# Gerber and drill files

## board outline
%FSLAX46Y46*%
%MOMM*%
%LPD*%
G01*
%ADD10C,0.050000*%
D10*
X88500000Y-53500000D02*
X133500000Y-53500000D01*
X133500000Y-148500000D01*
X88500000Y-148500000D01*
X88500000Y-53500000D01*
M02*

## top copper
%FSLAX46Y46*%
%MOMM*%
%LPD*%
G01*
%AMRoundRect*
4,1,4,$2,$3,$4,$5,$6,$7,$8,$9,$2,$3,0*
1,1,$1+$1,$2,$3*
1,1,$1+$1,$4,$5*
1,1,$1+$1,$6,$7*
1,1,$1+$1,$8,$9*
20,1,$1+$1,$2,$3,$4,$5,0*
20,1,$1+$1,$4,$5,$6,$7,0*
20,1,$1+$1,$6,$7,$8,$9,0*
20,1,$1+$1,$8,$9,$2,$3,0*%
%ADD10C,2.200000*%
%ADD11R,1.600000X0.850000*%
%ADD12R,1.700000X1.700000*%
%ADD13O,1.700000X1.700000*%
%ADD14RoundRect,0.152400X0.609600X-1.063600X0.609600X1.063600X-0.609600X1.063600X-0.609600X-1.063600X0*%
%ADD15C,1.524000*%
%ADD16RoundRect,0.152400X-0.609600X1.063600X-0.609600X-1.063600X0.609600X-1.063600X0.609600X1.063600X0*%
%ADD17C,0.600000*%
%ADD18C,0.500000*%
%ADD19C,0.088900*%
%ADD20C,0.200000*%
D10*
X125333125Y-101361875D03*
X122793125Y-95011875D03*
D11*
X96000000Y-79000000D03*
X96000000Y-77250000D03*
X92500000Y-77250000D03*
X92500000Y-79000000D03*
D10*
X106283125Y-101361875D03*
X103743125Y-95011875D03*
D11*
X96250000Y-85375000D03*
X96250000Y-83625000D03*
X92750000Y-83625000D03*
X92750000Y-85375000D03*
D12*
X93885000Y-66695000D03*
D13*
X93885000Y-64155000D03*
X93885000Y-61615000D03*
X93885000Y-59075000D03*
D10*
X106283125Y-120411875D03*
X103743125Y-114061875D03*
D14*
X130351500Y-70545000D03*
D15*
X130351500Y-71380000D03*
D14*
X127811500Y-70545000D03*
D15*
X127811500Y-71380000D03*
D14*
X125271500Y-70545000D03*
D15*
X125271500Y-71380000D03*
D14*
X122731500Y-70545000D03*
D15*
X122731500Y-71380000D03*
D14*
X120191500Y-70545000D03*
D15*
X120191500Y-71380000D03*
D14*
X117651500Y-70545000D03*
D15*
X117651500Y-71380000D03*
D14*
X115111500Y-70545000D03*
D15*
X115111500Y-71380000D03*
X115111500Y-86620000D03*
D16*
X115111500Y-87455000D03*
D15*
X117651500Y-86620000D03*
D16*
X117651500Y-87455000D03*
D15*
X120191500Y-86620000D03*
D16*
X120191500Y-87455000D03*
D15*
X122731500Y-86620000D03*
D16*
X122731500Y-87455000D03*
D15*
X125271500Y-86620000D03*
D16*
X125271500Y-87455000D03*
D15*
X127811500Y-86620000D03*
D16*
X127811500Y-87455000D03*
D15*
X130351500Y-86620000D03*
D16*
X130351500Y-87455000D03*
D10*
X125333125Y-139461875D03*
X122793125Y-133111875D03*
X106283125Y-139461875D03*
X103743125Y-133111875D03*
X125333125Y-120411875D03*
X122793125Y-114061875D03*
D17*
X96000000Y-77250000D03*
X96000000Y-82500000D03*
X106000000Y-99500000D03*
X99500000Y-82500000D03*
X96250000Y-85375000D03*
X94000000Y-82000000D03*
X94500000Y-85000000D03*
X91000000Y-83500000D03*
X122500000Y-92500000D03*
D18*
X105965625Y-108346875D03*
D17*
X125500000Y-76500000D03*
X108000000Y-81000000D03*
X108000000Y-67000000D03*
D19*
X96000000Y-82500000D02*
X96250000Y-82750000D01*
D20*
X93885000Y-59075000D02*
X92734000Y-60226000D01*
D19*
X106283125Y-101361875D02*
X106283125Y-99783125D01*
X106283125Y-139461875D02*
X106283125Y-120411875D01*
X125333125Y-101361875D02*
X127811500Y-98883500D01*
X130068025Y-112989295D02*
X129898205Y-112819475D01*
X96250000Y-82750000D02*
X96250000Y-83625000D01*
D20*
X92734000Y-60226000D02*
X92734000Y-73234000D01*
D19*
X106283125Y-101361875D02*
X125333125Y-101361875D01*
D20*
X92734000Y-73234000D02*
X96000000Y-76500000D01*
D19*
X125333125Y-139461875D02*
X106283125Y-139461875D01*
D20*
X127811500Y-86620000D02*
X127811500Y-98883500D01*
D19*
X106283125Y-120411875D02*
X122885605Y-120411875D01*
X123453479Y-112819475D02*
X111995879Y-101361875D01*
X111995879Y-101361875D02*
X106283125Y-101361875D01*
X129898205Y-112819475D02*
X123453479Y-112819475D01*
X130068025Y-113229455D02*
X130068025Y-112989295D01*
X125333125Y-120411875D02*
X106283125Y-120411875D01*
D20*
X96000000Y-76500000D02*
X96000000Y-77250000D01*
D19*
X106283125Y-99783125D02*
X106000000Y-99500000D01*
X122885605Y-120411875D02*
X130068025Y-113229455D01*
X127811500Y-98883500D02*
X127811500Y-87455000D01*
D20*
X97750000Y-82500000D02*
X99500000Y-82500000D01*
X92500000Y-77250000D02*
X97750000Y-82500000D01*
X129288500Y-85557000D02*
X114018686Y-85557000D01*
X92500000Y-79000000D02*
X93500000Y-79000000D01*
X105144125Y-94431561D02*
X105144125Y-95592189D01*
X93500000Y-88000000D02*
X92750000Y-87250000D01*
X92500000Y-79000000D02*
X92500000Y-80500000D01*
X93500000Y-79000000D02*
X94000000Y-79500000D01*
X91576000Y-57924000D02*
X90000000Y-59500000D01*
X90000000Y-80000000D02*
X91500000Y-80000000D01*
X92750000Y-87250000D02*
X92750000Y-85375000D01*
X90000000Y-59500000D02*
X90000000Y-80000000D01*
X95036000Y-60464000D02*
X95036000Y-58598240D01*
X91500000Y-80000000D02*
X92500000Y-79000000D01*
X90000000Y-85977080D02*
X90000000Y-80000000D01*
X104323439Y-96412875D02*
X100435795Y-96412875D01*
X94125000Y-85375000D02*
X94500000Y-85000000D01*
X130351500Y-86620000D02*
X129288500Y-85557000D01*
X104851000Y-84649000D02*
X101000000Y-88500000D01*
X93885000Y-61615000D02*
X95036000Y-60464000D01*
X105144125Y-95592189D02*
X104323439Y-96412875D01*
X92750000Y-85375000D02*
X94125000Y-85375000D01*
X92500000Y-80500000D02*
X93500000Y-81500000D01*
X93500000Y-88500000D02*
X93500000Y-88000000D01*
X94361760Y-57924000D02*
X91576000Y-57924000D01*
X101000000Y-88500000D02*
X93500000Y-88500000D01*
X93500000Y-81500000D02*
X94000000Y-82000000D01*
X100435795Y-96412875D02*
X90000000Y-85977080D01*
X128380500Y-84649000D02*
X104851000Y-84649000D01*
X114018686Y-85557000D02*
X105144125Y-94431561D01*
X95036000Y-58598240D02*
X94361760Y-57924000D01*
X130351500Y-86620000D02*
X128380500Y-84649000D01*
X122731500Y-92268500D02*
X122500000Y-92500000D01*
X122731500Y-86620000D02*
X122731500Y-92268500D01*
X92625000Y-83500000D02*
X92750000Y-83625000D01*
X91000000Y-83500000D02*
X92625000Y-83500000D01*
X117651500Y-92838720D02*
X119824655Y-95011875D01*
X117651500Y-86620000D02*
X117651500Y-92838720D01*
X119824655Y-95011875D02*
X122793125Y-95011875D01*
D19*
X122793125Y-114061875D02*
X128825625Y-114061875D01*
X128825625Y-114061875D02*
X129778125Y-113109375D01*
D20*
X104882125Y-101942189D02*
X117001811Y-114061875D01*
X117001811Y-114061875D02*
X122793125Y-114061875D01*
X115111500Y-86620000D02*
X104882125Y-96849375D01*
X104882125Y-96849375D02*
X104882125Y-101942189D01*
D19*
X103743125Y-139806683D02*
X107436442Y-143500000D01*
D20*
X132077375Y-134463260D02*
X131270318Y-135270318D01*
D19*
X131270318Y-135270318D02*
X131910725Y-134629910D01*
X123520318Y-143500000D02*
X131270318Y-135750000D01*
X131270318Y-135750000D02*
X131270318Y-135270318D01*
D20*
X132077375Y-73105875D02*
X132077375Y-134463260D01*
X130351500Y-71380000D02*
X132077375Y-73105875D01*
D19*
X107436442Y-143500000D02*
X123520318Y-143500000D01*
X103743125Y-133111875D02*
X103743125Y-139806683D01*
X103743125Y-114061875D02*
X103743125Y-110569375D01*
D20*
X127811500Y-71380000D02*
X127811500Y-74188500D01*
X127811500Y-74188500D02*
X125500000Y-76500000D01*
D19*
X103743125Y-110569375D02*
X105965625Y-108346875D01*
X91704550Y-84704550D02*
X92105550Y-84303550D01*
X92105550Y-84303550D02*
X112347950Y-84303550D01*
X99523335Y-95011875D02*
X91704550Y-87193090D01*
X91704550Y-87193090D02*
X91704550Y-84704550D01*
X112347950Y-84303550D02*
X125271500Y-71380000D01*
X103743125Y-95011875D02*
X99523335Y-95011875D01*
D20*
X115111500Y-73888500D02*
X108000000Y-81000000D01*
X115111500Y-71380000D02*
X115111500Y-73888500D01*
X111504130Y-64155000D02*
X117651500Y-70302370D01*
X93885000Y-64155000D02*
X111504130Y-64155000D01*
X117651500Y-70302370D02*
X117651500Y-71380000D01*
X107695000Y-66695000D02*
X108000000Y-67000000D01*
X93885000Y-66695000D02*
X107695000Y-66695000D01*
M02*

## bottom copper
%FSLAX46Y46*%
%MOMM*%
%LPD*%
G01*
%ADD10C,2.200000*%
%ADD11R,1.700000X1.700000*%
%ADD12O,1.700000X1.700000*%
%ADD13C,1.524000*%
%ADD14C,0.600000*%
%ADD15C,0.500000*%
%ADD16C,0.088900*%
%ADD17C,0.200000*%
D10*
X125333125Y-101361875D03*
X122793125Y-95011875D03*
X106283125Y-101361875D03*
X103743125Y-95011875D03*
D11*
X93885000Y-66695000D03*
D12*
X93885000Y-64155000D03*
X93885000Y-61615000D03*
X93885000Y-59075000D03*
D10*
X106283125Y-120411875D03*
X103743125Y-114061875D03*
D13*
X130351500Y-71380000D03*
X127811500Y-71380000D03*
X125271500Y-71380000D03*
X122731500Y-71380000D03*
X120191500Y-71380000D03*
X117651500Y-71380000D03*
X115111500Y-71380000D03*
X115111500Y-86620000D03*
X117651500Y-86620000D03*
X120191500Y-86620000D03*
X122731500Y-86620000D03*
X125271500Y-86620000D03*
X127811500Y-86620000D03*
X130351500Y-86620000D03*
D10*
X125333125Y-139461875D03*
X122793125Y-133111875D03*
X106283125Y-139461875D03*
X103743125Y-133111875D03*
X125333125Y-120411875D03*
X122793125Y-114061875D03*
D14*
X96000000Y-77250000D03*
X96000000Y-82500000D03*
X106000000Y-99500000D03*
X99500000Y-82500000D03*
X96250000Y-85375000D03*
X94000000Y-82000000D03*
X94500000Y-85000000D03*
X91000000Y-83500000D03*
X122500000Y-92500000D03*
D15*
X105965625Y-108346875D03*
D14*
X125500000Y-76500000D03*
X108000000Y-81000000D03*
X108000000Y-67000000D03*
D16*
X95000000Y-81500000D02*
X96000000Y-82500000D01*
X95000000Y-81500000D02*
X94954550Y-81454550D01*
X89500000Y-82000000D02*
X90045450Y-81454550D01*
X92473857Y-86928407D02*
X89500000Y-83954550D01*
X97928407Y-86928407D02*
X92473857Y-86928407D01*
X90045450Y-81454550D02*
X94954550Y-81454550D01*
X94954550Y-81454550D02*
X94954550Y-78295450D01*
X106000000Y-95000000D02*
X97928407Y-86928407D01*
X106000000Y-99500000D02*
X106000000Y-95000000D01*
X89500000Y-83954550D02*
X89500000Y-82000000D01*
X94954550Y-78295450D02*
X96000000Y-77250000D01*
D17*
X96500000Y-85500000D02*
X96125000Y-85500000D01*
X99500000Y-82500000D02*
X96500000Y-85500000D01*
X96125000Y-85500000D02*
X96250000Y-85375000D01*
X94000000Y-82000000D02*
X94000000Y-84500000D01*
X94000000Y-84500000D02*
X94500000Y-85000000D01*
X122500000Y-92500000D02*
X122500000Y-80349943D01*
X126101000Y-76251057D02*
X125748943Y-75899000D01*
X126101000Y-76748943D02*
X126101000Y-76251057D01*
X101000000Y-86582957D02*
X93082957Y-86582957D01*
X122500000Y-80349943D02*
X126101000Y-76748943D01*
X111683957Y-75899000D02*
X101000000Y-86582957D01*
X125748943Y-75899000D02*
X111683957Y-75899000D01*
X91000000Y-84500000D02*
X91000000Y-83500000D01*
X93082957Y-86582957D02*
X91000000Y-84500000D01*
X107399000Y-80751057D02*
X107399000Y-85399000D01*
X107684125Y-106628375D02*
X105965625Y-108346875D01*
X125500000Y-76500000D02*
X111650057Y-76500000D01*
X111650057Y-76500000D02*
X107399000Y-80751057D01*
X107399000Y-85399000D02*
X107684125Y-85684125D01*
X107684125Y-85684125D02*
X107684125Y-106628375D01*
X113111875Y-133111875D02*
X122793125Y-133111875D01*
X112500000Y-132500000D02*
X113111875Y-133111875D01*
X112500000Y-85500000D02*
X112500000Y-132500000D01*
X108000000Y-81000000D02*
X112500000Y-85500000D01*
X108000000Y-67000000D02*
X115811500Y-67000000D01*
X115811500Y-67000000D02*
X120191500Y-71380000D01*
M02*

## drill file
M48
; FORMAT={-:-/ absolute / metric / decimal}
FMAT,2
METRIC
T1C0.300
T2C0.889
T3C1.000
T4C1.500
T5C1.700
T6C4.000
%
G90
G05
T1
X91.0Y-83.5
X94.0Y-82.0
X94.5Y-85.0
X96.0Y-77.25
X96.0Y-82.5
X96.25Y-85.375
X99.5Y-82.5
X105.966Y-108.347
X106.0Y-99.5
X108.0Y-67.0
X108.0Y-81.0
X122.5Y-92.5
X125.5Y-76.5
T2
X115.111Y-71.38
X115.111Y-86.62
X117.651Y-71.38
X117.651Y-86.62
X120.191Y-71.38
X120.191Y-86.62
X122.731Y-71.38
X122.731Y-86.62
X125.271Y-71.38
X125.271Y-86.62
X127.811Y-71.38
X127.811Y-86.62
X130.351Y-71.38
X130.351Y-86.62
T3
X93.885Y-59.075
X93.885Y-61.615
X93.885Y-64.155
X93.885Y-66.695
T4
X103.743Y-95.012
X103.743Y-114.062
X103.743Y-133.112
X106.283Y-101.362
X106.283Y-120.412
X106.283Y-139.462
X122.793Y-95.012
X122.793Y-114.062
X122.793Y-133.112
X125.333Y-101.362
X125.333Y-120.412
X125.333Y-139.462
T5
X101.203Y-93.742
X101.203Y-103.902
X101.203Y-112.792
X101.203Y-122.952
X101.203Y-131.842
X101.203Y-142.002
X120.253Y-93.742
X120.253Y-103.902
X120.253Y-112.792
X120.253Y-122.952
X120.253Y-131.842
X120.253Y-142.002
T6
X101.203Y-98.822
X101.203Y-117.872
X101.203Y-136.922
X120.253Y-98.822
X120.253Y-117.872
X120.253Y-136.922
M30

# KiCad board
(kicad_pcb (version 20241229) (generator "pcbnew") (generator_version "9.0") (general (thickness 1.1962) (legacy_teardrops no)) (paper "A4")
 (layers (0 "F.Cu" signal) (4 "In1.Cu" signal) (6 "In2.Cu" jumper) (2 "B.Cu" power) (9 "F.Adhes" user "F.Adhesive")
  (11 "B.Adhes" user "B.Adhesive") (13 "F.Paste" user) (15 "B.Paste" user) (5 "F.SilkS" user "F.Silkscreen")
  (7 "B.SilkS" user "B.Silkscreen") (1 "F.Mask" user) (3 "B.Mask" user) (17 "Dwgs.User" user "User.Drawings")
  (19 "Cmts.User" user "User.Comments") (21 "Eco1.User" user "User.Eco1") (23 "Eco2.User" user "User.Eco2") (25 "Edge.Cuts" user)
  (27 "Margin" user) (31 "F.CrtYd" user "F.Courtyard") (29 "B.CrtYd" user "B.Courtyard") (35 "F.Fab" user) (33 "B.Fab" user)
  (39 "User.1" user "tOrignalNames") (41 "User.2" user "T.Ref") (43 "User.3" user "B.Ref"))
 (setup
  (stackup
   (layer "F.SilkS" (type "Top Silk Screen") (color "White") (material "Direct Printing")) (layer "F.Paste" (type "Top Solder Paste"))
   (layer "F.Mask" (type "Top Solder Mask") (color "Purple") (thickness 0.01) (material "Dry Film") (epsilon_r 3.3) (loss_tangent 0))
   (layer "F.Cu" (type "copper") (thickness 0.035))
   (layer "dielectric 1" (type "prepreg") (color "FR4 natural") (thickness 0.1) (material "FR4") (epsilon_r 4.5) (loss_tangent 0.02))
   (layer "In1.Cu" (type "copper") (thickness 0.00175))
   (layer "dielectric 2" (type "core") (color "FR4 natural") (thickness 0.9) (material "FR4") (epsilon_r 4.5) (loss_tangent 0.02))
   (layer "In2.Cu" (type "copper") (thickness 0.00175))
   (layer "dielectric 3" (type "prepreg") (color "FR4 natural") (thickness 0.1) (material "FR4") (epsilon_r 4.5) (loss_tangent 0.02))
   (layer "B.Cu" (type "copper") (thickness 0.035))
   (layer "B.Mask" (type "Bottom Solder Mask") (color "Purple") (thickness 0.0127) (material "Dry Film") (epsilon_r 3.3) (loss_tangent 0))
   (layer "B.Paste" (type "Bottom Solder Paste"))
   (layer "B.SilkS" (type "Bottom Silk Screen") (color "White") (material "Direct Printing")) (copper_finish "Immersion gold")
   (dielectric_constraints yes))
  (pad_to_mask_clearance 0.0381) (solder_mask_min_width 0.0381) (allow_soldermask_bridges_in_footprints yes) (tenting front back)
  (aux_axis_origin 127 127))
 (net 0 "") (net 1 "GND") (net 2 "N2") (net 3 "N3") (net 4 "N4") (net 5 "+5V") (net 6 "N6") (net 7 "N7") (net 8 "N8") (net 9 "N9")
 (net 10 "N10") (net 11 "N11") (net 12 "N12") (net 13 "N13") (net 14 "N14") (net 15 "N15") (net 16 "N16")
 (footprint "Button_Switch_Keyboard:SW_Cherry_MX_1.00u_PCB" (layer "F.Cu") (at 125.333125 101.361875 -90)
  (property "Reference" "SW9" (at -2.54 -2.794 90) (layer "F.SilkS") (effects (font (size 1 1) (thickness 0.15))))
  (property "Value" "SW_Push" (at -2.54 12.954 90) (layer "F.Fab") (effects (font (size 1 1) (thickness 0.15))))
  (pad "" np_thru_hole circle (at -7.62 5.08 270) (size 1.7 1.7) (drill 1.7) (layers "*.Cu" "*.Mask"))
  (pad "" np_thru_hole circle (at -2.54 5.08 270) (size 4 4) (drill 4) (layers "*.Cu" "*.Mask"))
  (pad "" np_thru_hole circle (at 2.54 5.08 270) (size 1.7 1.7) (drill 1.7) (layers "*.Cu" "*.Mask"))
  (pad "1" thru_hole circle (at 0 0 270) (size 2.2 2.2) (drill 1.5) (layers "*.Cu" "*.Mask") (remove_unused_layers no) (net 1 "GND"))
  (pad "2" thru_hole circle (at -6.35 2.54 270) (size 2.2 2.2) (drill 1.5) (layers "*.Cu" "*.Mask") (remove_unused_layers no) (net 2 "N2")))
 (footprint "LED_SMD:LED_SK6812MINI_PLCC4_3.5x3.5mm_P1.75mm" (layer "F.Cu") (at 94.25 78.125 180)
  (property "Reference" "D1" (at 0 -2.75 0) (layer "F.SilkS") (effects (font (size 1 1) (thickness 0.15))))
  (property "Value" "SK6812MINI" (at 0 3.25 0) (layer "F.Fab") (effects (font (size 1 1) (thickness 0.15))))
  (pad "1" smd rect (at -1.75 -0.875 180) (size 1.6 0.85) (layers "F.Cu" "F.Mask" "F.Paste") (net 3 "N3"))
  (pad "2" smd rect (at -1.75 0.875 180) (size 1.6 0.85) (layers "F.Cu" "F.Mask" "F.Paste") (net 1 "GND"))
  (pad "3" smd rect (at 1.75 0.875 180) (size 1.6 0.85) (layers "F.Cu" "F.Mask" "F.Paste") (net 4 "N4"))
  (pad "4" smd rect (at 1.75 -0.875 180) (size 1.6 0.85) (layers "F.Cu" "F.Mask" "F.Paste") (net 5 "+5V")))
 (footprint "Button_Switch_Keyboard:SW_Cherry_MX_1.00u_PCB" (layer "F.Cu") (at 106.283125 101.361875 -90)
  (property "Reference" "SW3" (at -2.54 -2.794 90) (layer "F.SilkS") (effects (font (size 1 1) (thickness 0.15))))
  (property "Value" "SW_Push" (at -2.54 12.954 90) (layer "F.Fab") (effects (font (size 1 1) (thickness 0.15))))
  (pad "" np_thru_hole circle (at -7.62 5.08 270) (size 1.7 1.7) (drill 1.7) (layers "*.Cu" "*.Mask"))
  (pad "" np_thru_hole circle (at -2.54 5.08 270) (size 4 4) (drill 4) (layers "*.Cu" "*.Mask"))
  (pad "" np_thru_hole circle (at 2.54 5.08 270) (size 1.7 1.7) (drill 1.7) (layers "*.Cu" "*.Mask"))
  (pad "1" thru_hole circle (at 0 0 270) (size 2.2 2.2) (drill 1.5) (layers "*.Cu" "*.Mask") (remove_unused_layers no) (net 1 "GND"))
  (pad "2" thru_hole circle (at -6.35 2.54 270) (size 2.2 2.2) (drill 1.5) (layers "*.Cu" "*.Mask") (remove_unused_layers no) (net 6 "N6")))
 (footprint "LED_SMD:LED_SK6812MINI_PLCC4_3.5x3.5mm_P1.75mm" (layer "F.Cu") (at 94.5 84.5 180)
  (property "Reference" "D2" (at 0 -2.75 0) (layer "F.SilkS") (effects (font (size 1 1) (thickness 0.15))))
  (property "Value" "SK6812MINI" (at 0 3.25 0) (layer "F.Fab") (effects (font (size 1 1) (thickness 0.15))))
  (pad "1" smd rect (at -1.75 -0.875 180) (size 1.6 0.85) (layers "F.Cu" "F.Mask" "F.Paste") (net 4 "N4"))
  (pad "2" smd rect (at -1.75 0.875 180) (size 1.6 0.85) (layers "F.Cu" "F.Mask" "F.Paste") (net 1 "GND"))
  (pad "3" smd rect (at 1.75 0.875 180) (size 1.6 0.85) (layers "F.Cu" "F.Mask" "F.Paste") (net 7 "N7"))
  (pad "4" smd rect (at 1.75 -0.875 180) (size 1.6 0.85) (layers "F.Cu" "F.Mask" "F.Paste") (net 5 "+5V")))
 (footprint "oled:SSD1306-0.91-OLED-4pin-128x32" (layer "F.Cu") (at 130.385 68.885 180)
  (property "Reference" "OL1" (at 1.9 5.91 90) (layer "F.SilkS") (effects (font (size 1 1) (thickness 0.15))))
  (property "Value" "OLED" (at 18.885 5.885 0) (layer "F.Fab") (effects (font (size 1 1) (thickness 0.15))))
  (pad "1" thru_hole rect (at 36.5 2.19 180) (size 1.7 1.7) (drill 1) (layers "*.Cu" "*.Mask") (remove_unused_layers no) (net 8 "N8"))
  (pad "2" thru_hole oval (at 36.5 4.73 180) (size 1.7 1.7) (drill 1) (layers "*.Cu" "*.Mask") (remove_unused_layers no) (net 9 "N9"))
  (pad "3" thru_hole oval (at 36.5 7.27 180) (size 1.7 1.7) (drill 1) (layers "*.Cu" "*.Mask") (remove_unused_layers no) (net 5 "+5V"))
  (pad "4" thru_hole oval (at 36.5 9.81 180) (size 1.7 1.7) (drill 1) (layers "*.Cu" "*.Mask") (remove_unused_layers no) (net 1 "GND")))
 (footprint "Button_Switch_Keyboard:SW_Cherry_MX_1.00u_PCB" (layer "F.Cu") (at 106.283125 120.411875 -90)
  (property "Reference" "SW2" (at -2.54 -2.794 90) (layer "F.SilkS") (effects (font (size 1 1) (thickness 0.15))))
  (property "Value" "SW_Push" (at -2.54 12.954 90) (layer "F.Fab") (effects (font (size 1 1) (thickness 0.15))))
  (pad "" np_thru_hole circle (at -7.62 5.08 270) (size 1.7 1.7) (drill 1.7) (layers "*.Cu" "*.Mask"))
  (pad "" np_thru_hole circle (at -2.54 5.08 270) (size 4 4) (drill 4) (layers "*.Cu" "*.Mask"))
  (pad "" np_thru_hole circle (at 2.54 5.08 270) (size 1.7 1.7) (drill 1.7) (layers "*.Cu" "*.Mask"))
  (pad "1" thru_hole circle (at 0 0 270) (size 2.2 2.2) (drill 1.5) (layers "*.Cu" "*.Mask") (remove_unused_layers no) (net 1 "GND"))
  (pad "2" thru_hole circle (at -6.35 2.54 270) (size 2.2 2.2) (drill 1.5) (layers "*.Cu" "*.Mask") (remove_unused_layers no) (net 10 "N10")))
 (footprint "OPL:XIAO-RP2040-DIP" (layer "F.Cu") (at 122.7315 79 -90)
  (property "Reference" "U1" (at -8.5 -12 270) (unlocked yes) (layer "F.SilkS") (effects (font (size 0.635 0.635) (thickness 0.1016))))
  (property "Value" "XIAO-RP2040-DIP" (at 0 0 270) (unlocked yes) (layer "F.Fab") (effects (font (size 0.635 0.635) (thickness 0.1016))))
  (pad "1" smd roundrect (at -8.455 -7.62 90) (size 2.432 1.524) (layers "F.Cu" "F.Mask") (roundrect_rratio 0.1) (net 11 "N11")
   (thermal_bridge_angle 45))
  (pad "1" thru_hole circle (at -7.62 -7.62 90) (size 1.524 1.524) (drill 0.889) (layers "*.Cu" "*.Mask") (remove_unused_layers no)
   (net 11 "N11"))
  (pad "2" smd roundrect (at -8.455 -5.08 90) (size 2.432 1.524) (layers "F.Cu" "F.Mask") (roundrect_rratio 0.1) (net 10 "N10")
   (thermal_bridge_angle 45))
  (pad "2" thru_hole circle (at -7.62 -5.08 90) (size 1.524 1.524) (drill 0.889) (layers "*.Cu" "*.Mask") (remove_unused_layers no)
   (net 10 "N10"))
  (pad "3" smd roundrect (at -8.455 -2.54 90) (size 2.432 1.524) (layers "F.Cu" "F.Mask") (roundrect_rratio 0.1) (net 6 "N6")
   (thermal_bridge_angle 45))
  (pad "3" thru_hole circle (at -7.62 -2.54 90) (size 1.524 1.524) (drill 0.889) (layers "*.Cu" "*.Mask") (remove_unused_layers no)
   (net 6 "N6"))
  (pad "4" smd roundrect (at -8.455 0 90) (size 2.432 1.524) (layers "F.Cu" "F.Mask") (roundrect_rratio 0.1) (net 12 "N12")
   (thermal_bridge_angle 45))
  (pad "4" thru_hole circle (at -7.62 0 90) (size 1.524 1.524) (drill 0.889) (layers "*.Cu" "*.Mask") (remove_unused_layers no)
   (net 12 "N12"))
  (pad "5" smd roundrect (at -8.455 2.54 90) (size 2.432 1.524) (layers "F.Cu" "F.Mask") (roundrect_rratio 0.1) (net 8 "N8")
   (thermal_bridge_angle 45))
  (pad "5" thru_hole circle (at -7.62 2.54 90) (size 1.524 1.524) (drill 0.889) (layers "*.Cu" "*.Mask") (remove_unused_layers no)
   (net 8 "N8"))
  (pad "6" smd roundrect (at -8.455 5.08 90) (size 2.432 1.524) (layers "F.Cu" "F.Mask") (roundrect_rratio 0.1) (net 9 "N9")
   (thermal_bridge_angle 45))
  (pad "6" thru_hole circle (at -7.62 5.08 90) (size 1.524 1.524) (drill 0.889) (layers "*.Cu" "*.Mask") (remove_unused_layers no)
   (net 9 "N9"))
  (pad "7" smd roundrect (at -8.455 7.62 90) (size 2.432 1.524) (layers "F.Cu" "F.Mask") (roundrect_rratio 0.1) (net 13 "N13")
   (thermal_bridge_angle 45))
  (pad "7" thru_hole circle (at -7.62 7.62 90) (size 1.524 1.524) (drill 0.889) (layers "*.Cu" "*.Mask") (remove_unused_layers no)
   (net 13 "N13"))
  (pad "8" thru_hole circle (at 7.62 7.62 270) (size 1.524 1.524) (drill 0.889) (layers "*.Cu" "*.Mask") (remove_unused_layers no)
   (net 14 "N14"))
  (pad "8" smd roundrect (at 8.455 7.62 270) (size 2.432 1.524) (layers "F.Cu" "F.Mask") (roundrect_rratio 0.1) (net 14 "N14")
   (thermal_bridge_angle 45))
  (pad "9" thru_hole circle (at 7.62 5.08 270) (size 1.524 1.524) (drill 0.889) (layers "*.Cu" "*.Mask") (remove_unused_layers no)
   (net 2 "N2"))
  (pad "9" smd roundrect (at 8.455 5.08 270) (size 2.432 1.524) (layers "F.Cu" "F.Mask") (roundrect_rratio 0.1) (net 2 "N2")
   (thermal_bridge_angle 45))
  (pad "10" thru_hole circle (at 7.62 2.54 270) (size 1.524 1.524) (drill 0.889) (layers "*.Cu" "*.Mask") (remove_unused_layers no)
   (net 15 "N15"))
  (pad "10" smd roundrect (at 8.455 2.54 270) (size 2.432 1.524) (layers "F.Cu" "F.Mask") (roundrect_rratio 0.1) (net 15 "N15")
   (thermal_bridge_angle 45))
  (pad "11" thru_hole circle (at 7.62 0 270) (size 1.524 1.524) (drill 0.889) (layers "*.Cu" "*.Mask") (remove_unused_layers no)
   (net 7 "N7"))
  (pad "11" smd roundrect (at 8.455 0 270) (size 2.432 1.524) (layers "F.Cu" "F.Mask") (roundrect_rratio 0.1) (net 7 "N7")
   (thermal_bridge_angle 45))
  (pad "12" thru_hole circle (at 7.62 -2.54 270) (size 1.524 1.524) (drill 0.889) (layers "*.Cu" "*.Mask") (remove_unused_layers no)
   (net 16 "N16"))
  (pad "12" smd roundrect (at 8.455 -2.54 270) (size 2.432 1.524) (layers "F.Cu" "F.Mask") (roundrect_rratio 0.1) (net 16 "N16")
   (thermal_bridge_angle 45))
  (pad "13" thru_hole circle (at 7.62 -5.08 270) (size 1.524 1.524) (drill 0.889) (layers "*.Cu" "*.Mask") (remove_unused_layers no)
   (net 1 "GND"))
  (pad "13" smd roundrect (at 8.455 -5.08 270) (size 2.432 1.524) (layers "F.Cu" "F.Mask") (roundrect_rratio 0.1) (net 1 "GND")
   (thermal_bridge_angle 45))
  (pad "14" thru_hole circle (at 7.62 -7.62 270) (size 1.524 1.524) (drill 0.889) (layers "*.Cu" "*.Mask") (remove_unused_layers no)
   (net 5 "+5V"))
  (pad "14" smd roundrect (at 8.455 -7.62 270) (size 2.432 1.524) (layers "F.Cu" "F.Mask") (roundrect_rratio 0.1) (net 5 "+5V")
   (thermal_bridge_angle 45)))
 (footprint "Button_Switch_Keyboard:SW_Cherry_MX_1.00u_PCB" (layer "F.Cu") (at 125.333125 139.461875 -90)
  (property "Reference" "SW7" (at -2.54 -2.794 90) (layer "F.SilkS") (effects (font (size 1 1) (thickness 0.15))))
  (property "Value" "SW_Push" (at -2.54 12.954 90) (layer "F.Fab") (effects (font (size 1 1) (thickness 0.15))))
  (pad "" np_thru_hole circle (at -7.62 5.08 270) (size 1.7 1.7) (drill 1.7) (layers "*.Cu" "*.Mask"))
  (pad "" np_thru_hole circle (at -2.54 5.08 270) (size 4 4) (drill 4) (layers "*.Cu" "*.Mask"))
  (pad "" np_thru_hole circle (at 2.54 5.08 270) (size 1.7 1.7) (drill 1.7) (layers "*.Cu" "*.Mask"))
  (pad "1" thru_hole circle (at 0 0 270) (size 2.2 2.2) (drill 1.5) (layers "*.Cu" "*.Mask") (remove_unused_layers no) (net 1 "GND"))
  (pad "2" thru_hole circle (at -6.35 2.54 270) (size 2.2 2.2) (drill 1.5) (layers "*.Cu" "*.Mask") (remove_unused_layers no) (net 13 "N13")))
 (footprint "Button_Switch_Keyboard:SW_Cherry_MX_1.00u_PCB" (layer "F.Cu") (at 106.283125 139.461875 -90)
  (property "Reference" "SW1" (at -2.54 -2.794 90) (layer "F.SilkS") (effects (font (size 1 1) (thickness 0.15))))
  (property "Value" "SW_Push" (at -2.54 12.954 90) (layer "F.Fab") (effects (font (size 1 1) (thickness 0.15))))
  (pad "" np_thru_hole circle (at -7.62 5.08 270) (size 1.7 1.7) (drill 1.7) (layers "*.Cu" "*.Mask"))
  (pad "" np_thru_hole circle (at -2.54 5.08 270) (size 4 4) (drill 4) (layers "*.Cu" "*.Mask"))
  (pad "" np_thru_hole circle (at 2.54 5.08 270) (size 1.7 1.7) (drill 1.7) (layers "*.Cu" "*.Mask"))
  (pad "1" thru_hole circle (at 0 0 270) (size 2.2 2.2) (drill 1.5) (layers "*.Cu" "*.Mask") (remove_unused_layers no) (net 1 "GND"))
  (pad "2" thru_hole circle (at -6.35 2.54 270) (size 2.2 2.2) (drill 1.5) (layers "*.Cu" "*.Mask") (remove_unused_layers no) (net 11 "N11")))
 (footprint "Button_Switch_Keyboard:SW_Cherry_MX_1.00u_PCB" (layer "F.Cu") (at 125.333125 120.411875 -90)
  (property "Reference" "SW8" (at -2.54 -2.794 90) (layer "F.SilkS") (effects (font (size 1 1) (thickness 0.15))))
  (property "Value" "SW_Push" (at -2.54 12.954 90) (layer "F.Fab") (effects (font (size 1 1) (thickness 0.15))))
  (pad "" np_thru_hole circle (at -7.62 5.08 270) (size 1.7 1.7) (drill 1.7) (layers "*.Cu" "*.Mask"))
  (pad "" np_thru_hole circle (at -2.54 5.08 270) (size 4 4) (drill 4) (layers "*.Cu" "*.Mask"))
  (pad "" np_thru_hole circle (at 2.54 5.08 270) (size 1.7 1.7) (drill 1.7) (layers "*.Cu" "*.Mask"))
  (pad "1" thru_hole circle (at 0 0 270) (size 2.2 2.2) (drill 1.5) (layers "*.Cu" "*.Mask") (remove_unused_layers no) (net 1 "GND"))
  (pad "2" thru_hole circle (at -6.35 2.54 270) (size 2.2 2.2) (drill 1.5) (layers "*.Cu" "*.Mask") (remove_unused_layers no) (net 14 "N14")))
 (gr_rect (start 88.5 53.5) (end 133.5 148.5) (stroke (width 0.05) (type default)) (fill no) (layer "Edge.Cuts"))
 (segment (start 96 82.5) (end 96.25 82.75) (width 0.0889) (layer "F.Cu") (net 1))
 (segment (start 93.885 59.075) (end 92.734 60.226) (width 0.2) (layer "F.Cu") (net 1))
 (segment (start 106.283125 101.361875) (end 106.283125 99.783125) (width 0.0889) (layer "F.Cu") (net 1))
 (segment (start 106.283125 139.461875) (end 106.283125 120.411875) (width 0.0889) (layer "F.Cu") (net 1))
 (segment (start 125.333125 101.361875) (end 127.8115 98.8835) (width 0.0889) (layer "F.Cu") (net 1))
 (segment (start 130.068025 112.989295) (end 129.898205 112.819475) (width 0.0889) (layer "F.Cu") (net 1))
 (segment (start 96.25 82.75) (end 96.25 83.625) (width 0.0889) (layer "F.Cu") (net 1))
 (segment (start 92.734 60.226) (end 92.734 73.234) (width 0.2) (layer "F.Cu") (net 1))
 (segment (start 106.283125 101.361875) (end 125.333125 101.361875) (width 0.0889) (layer "F.Cu") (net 1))
 (segment (start 92.734 73.234) (end 96 76.5) (width 0.2) (layer "F.Cu") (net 1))
 (segment (start 125.333125 139.461875) (end 106.283125 139.461875) (width 0.0889) (layer "F.Cu") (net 1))
 (segment (start 127.8115 86.62) (end 127.8115 98.8835) (width 0.2) (layer "F.Cu") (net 1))
 (segment (start 106.283125 120.411875) (end 122.885605 120.411875) (width 0.0889) (layer "F.Cu") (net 1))
 (segment (start 123.453479 112.819475) (end 111.995879 101.361875) (width 0.0889) (layer "F.Cu") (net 1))
 (segment (start 111.995879 101.361875) (end 106.283125 101.361875) (width 0.0889) (layer "F.Cu") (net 1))
 (segment (start 129.898205 112.819475) (end 123.453479 112.819475) (width 0.0889) (layer "F.Cu") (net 1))
 (segment (start 130.068025 113.229455) (end 130.068025 112.989295) (width 0.0889) (layer "F.Cu") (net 1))
 (segment (start 125.333125 120.411875) (end 106.283125 120.411875) (width 0.0889) (layer "F.Cu") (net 1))
 (segment (start 96 76.5) (end 96 77.25) (width 0.2) (layer "F.Cu") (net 1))
 (segment (start 106.283125 99.783125) (end 106 99.5) (width 0.0889) (layer "F.Cu") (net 1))
 (segment (start 122.885605 120.411875) (end 130.068025 113.229455) (width 0.0889) (layer "F.Cu") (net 1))
 (segment (start 127.8115 98.8835) (end 127.8115 87.455) (width 0.0889) (layer "F.Cu") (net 1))
 (via (at 96 77.25) (size 0.6) (drill 0.3) (layers "F.Cu" "B.Cu") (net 1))
 (via (at 96 82.5) (size 0.6) (drill 0.3) (layers "F.Cu" "B.Cu") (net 1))
 (via (at 106 99.5) (size 0.6) (drill 0.3) (layers "F.Cu" "B.Cu") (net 1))
 (segment (start 95 81.5) (end 96 82.5) (width 0.0889) (layer "B.Cu") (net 1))
 (segment (start 95 81.5) (end 94.95455 81.45455) (width 0.0889) (layer "B.Cu") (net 1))
 (segment (start 89.5 82) (end 90.04545 81.45455) (width 0.0889) (layer "B.Cu") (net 1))
 (segment (start 92.473857 86.928407) (end 89.5 83.95455) (width 0.0889) (layer "B.Cu") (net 1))
 (segment (start 97.928407 86.928407) (end 92.473857 86.928407) (width 0.0889) (layer "B.Cu") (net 1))
 (segment (start 90.04545 81.45455) (end 94.95455 81.45455) (width 0.0889) (layer "B.Cu") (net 1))
 (segment (start 94.95455 81.45455) (end 94.95455 78.29545) (width 0.0889) (layer "B.Cu") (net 1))
 (segment (start 106 95) (end 97.928407 86.928407) (width 0.0889) (layer "B.Cu") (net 1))
 (segment (start 106 99.5) (end 106 95) (width 0.0889) (layer "B.Cu") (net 1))
 (segment (start 89.5 83.95455) (end 89.5 82) (width 0.0889) (layer "B.Cu") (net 1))
 (segment (start 94.95455 78.29545) (end 96 77.25) (width 0.0889) (layer "B.Cu") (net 1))
 (segment (start 97.75 82.5) (end 99.5 82.5) (width 0.2) (layer "F.Cu") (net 4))
 (segment (start 92.5 77.25) (end 97.75 82.5) (width 0.2) (layer "F.Cu") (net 4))
 (via (at 99.5 82.5) (size 0.6) (drill 0.3) (layers "F.Cu" "B.Cu") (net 4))
 (via (at 96.25 85.375) (size 0.6) (drill 0.3) (layers "F.Cu" "B.Cu") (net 4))
 (segment (start 96.5 85.5) (end 96.125 85.5) (width 0.2) (layer "B.Cu") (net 4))
 (segment (start 99.5 82.5) (end 96.5 85.5) (width 0.2) (layer "B.Cu") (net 4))
 (segment (start 96.125 85.5) (end 96.25 85.375) (width 0.2) (layer "B.Cu") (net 4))
 (segment (start 129.2885 85.557) (end 114.018686 85.557) (width 0.2) (layer "F.Cu") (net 5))
 (segment (start 92.5 79) (end 93.5 79) (width 0.2) (layer "F.Cu") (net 5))
 (segment (start 105.144125 94.431561) (end 105.144125 95.592189) (width 0.2) (layer "F.Cu") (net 5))
 (segment (start 93.5 88) (end 92.75 87.25) (width 0.2) (layer "F.Cu") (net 5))
 (segment (start 92.5 79) (end 92.5 80.5) (width 0.2) (layer "F.Cu") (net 5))
 (segment (start 93.5 79) (end 94 79.5) (width 0.2) (layer "F.Cu") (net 5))
 (segment (start 91.576 57.924) (end 90 59.5) (width 0.2) (layer "F.Cu") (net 5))
 (segment (start 90 80) (end 91.5 80) (width 0.2) (layer "F.Cu") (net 5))
 (segment (start 92.75 87.25) (end 92.75 85.375) (width 0.2) (layer "F.Cu") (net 5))
 (segment (start 90 59.5) (end 90 80) (width 0.2) (layer "F.Cu") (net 5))
 (segment (start 95.036 60.464) (end 95.036 58.59824) (width 0.2) (layer "F.Cu") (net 5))
 (segment (start 91.5 80) (end 92.5 79) (width 0.2) (layer "F.Cu") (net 5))
 (segment (start 90 85.97708) (end 90 80) (width 0.2) (layer "F.Cu") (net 5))
 (segment (start 104.323439 96.412875) (end 100.435795 96.412875) (width 0.2) (layer "F.Cu") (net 5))
 (segment (start 94.125 85.375) (end 94.5 85) (width 0.2) (layer "F.Cu") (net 5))
 (segment (start 130.3515 86.62) (end 129.2885 85.557) (width 0.2) (layer "F.Cu") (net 5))
 (segment (start 104.851 84.649) (end 101 88.5) (width 0.2) (layer "F.Cu") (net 5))
 (segment (start 93.885 61.615) (end 95.036 60.464) (width 0.2) (layer "F.Cu") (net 5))
 (segment (start 105.144125 95.592189) (end 104.323439 96.412875) (width 0.2) (layer "F.Cu") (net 5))
 (segment (start 92.75 85.375) (end 94.125 85.375) (width 0.2) (layer "F.Cu") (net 5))
 (segment (start 92.5 80.5) (end 93.5 81.5) (width 0.2) (layer "F.Cu") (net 5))
 (segment (start 93.5 88.5) (end 93.5 88) (width 0.2) (layer "F.Cu") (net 5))
 (segment (start 94.36176 57.924) (end 91.576 57.924) (width 0.2) (layer "F.Cu") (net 5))
 (segment (start 101 88.5) (end 93.5 88.5) (width 0.2) (layer "F.Cu") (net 5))
 (segment (start 93.5 81.5) (end 94 82) (width 0.2) (layer "F.Cu") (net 5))
 (segment (start 100.435795 96.412875) (end 90 85.97708) (width 0.2) (layer "F.Cu") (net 5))
 (segment (start 128.3805 84.649) (end 104.851 84.649) (width 0.2) (layer "F.Cu") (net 5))
 (segment (start 114.018686 85.557) (end 105.144125 94.431561) (width 0.2) (layer "F.Cu") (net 5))
 (segment (start 95.036 58.59824) (end 94.36176 57.924) (width 0.2) (layer "F.Cu") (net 5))
 (segment (start 130.3515 86.62) (end 128.3805 84.649) (width 0.2) (layer "F.Cu") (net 5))
 (via (at 94 82) (size 0.6) (drill 0.3) (layers "F.Cu" "B.Cu") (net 5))
 (via (at 94.5 85) (size 0.6) (drill 0.3) (layers "F.Cu" "B.Cu") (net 5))
 (segment (start 94 82) (end 94 84.5) (width 0.2) (layer "B.Cu") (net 5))
 (segment (start 94 84.5) (end 94.5 85) (width 0.2) (layer "B.Cu") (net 5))
 (segment (start 122.7315 92.2685) (end 122.5 92.5) (width 0.2) (layer "F.Cu") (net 7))
 (segment (start 122.7315 86.62) (end 122.7315 92.2685) (width 0.2) (layer "F.Cu") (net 7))
 (segment (start 92.625 83.5) (end 92.75 83.625) (width 0.2) (layer "F.Cu") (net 7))
 (segment (start 91 83.5) (end 92.625 83.5) (width 0.2) (layer "F.Cu") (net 7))
 (via (at 91 83.5) (size 0.6) (drill 0.3) (layers "F.Cu" "B.Cu") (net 7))
 (via (at 122.5 92.5) (size 0.6) (drill 0.3) (layers "F.Cu" "B.Cu") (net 7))
 (segment (start 122.5 92.5) (end 122.5 80.349943) (width 0.2) (layer "B.Cu") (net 7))
 (segment (start 126.101 76.251057) (end 125.748943 75.899) (width 0.2) (layer "B.Cu") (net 7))
 (segment (start 126.101 76.748943) (end 126.101 76.251057) (width 0.2) (layer "B.Cu") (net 7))
 (segment (start 101 86.582957) (end 93.082957 86.582957) (width 0.2) (layer "B.Cu") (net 7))
 (segment (start 122.5 80.349943) (end 126.101 76.748943) (width 0.2) (layer "B.Cu") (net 7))
 (segment (start 111.683957 75.899) (end 101 86.582957) (width 0.2) (layer "B.Cu") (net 7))
 (segment (start 125.748943 75.899) (end 111.683957 75.899) (width 0.2) (layer "B.Cu") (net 7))
 (segment (start 91 84.5) (end 91 83.5) (width 0.2) (layer "B.Cu") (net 7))
 (segment (start 93.082957 86.582957) (end 91 84.5) (width 0.2) (layer "B.Cu") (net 7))
 (segment (start 117.6515 92.83872) (end 119.824655 95.011875) (width 0.2) (layer "F.Cu") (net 2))
 (segment (start 117.6515 86.62) (end 117.6515 92.83872) (width 0.2) (layer "F.Cu") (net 2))
 (segment (start 119.824655 95.011875) (end 122.793125 95.011875) (width 0.2) (layer "F.Cu") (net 2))
 (segment (start 122.793125 114.061875) (end 128.825625 114.061875) (width 0.0889) (layer "F.Cu") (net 14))
 (segment (start 128.825625 114.061875) (end 129.778125 113.109375) (width 0.0889) (layer "F.Cu") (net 14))
 (segment (start 104.882125 101.942189) (end 117.001811 114.061875) (width 0.2) (layer "F.Cu") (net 14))
 (segment (start 117.001811 114.061875) (end 122.793125 114.061875) (width 0.2) (layer "F.Cu") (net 14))
 (segment (start 115.1115 86.62) (end 104.882125 96.849375) (width 0.2) (layer "F.Cu") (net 14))
 (segment (start 104.882125 96.849375) (end 104.882125 101.942189) (width 0.2) (layer "F.Cu") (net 14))
 (segment (start 103.743125 139.806683) (end 107.436442 143.5) (width 0.0889) (layer "F.Cu") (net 11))
 (segment (start 132.077375 134.46326) (end 131.270318 135.270318) (width 0.2) (layer "F.Cu") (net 11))
 (segment (start 131.270318 135.270318) (end 131.910725 134.62991) (width 0.0889) (layer "F.Cu") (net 11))
 (segment (start 123.520318 143.5) (end 131.270318 135.75) (width 0.0889) (layer "F.Cu") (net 11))
 (segment (start 131.270318 135.75) (end 131.270318 135.270318) (width 0.0889) (layer "F.Cu") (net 11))
 (segment (start 132.077375 73.105875) (end 132.077375 134.46326) (width 0.2) (layer "F.Cu") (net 11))
 (segment (start 130.3515 71.38) (end 132.077375 73.105875) (width 0.2) (layer "F.Cu") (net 11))
 (segment (start 107.436442 143.5) (end 123.520318 143.5) (width 0.0889) (layer "F.Cu") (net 11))
 (segment (start 103.743125 133.111875) (end 103.743125 139.806683) (width 0.0889) (layer "F.Cu") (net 11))
 (segment (start 103.743125 114.061875) (end 103.743125 110.569375) (width 0.0889) (layer "F.Cu") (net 10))
 (segment (start 127.8115 71.38) (end 127.8115 74.1885) (width 0.2) (layer "F.Cu") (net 10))
 (segment (start 127.8115 74.1885) (end 125.5 76.5) (width 0.2) (layer "F.Cu") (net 10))
 (segment (start 103.743125 110.569375) (end 105.965625 108.346875) (width 0.0889) (layer "F.Cu") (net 10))
 (via (at 105.965625 108.346875) (size 0.5) (drill 0.3) (layers "F.Cu" "B.Cu") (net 10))
 (via (at 125.5 76.5) (size 0.6) (drill 0.3) (layers "F.Cu" "B.Cu") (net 10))
 (segment (start 107.399 80.751057) (end 107.399 85.399) (width 0.2) (layer "B.Cu") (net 10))
 (segment (start 107.684125 106.628375) (end 105.965625 108.346875) (width 0.2) (layer "B.Cu") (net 10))
 (segment (start 125.5 76.5) (end 111.650057 76.5) (width 0.2) (layer "B.Cu") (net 10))
 (segment (start 111.650057 76.5) (end 107.399 80.751057) (width 0.2) (layer "B.Cu") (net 10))
 (segment (start 107.399 85.399) (end 107.684125 85.684125) (width 0.2) (layer "B.Cu") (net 10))
 (segment (start 107.684125 85.684125) (end 107.684125 106.628375) (width 0.2) (layer "B.Cu") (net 10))
 (segment (start 91.70455 84.70455) (end 92.10555 84.30355) (width 0.0889) (layer "F.Cu") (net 6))
 (segment (start 92.10555 84.30355) (end 112.34795 84.30355) (width 0.0889) (layer "F.Cu") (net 6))
 (segment (start 99.523335 95.011875) (end 91.70455 87.19309) (width 0.0889) (layer "F.Cu") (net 6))
 (segment (start 91.70455 87.19309) (end 91.70455 84.70455) (width 0.0889) (layer "F.Cu") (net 6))
 (segment (start 112.34795 84.30355) (end 125.2715 71.38) (width 0.0889) (layer "F.Cu") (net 6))
 (segment (start 103.743125 95.011875) (end 99.523335 95.011875) (width 0.0889) (layer "F.Cu") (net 6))
 (segment (start 115.1115 73.8885) (end 108 81) (width 0.2) (layer "F.Cu") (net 13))
 (segment (start 115.1115 71.38) (end 115.1115 73.8885) (width 0.2) (layer "F.Cu") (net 13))
 (via (at 108 81) (size 0.6) (drill 0.3) (layers "F.Cu" "B.Cu") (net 13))
 (segment (start 113.111875 133.111875) (end 122.793125 133.111875) (width 0.2) (layer "B.Cu") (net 13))
 (segment (start 112.5 132.5) (end 113.111875 133.111875) (width 0.2) (layer "B.Cu") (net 13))
 (segment (start 112.5 85.5) (end 112.5 132.5) (width 0.2) (layer "B.Cu") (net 13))
 (segment (start 108 81) (end 112.5 85.5) (width 0.2) (layer "B.Cu") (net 13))
 (segment (start 111.50413 64.155) (end 117.6515 70.30237) (width 0.2) (layer "F.Cu") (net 9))
 (segment (start 93.885 64.155) (end 111.50413 64.155) (width 0.2) (layer "F.Cu") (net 9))
 (segment (start 117.6515 70.30237) (end 117.6515 71.38) (width 0.2) (layer "F.Cu") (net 9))
 (segment (start 107.695 66.695) (end 108 67) (width 0.2) (layer "F.Cu") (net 8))
 (segment (start 93.885 66.695) (end 107.695 66.695) (width 0.2) (layer "F.Cu") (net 8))
 (via (at 108 67) (size 0.6) (drill 0.3) (layers "F.Cu" "B.Cu") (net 8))
 (segment (start 108 67) (end 115.8115 67) (width 0.2) (layer "B.Cu") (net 8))
 (segment (start 115.8115 67) (end 120.1915 71.38) (width 0.2) (layer "B.Cu") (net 8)))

